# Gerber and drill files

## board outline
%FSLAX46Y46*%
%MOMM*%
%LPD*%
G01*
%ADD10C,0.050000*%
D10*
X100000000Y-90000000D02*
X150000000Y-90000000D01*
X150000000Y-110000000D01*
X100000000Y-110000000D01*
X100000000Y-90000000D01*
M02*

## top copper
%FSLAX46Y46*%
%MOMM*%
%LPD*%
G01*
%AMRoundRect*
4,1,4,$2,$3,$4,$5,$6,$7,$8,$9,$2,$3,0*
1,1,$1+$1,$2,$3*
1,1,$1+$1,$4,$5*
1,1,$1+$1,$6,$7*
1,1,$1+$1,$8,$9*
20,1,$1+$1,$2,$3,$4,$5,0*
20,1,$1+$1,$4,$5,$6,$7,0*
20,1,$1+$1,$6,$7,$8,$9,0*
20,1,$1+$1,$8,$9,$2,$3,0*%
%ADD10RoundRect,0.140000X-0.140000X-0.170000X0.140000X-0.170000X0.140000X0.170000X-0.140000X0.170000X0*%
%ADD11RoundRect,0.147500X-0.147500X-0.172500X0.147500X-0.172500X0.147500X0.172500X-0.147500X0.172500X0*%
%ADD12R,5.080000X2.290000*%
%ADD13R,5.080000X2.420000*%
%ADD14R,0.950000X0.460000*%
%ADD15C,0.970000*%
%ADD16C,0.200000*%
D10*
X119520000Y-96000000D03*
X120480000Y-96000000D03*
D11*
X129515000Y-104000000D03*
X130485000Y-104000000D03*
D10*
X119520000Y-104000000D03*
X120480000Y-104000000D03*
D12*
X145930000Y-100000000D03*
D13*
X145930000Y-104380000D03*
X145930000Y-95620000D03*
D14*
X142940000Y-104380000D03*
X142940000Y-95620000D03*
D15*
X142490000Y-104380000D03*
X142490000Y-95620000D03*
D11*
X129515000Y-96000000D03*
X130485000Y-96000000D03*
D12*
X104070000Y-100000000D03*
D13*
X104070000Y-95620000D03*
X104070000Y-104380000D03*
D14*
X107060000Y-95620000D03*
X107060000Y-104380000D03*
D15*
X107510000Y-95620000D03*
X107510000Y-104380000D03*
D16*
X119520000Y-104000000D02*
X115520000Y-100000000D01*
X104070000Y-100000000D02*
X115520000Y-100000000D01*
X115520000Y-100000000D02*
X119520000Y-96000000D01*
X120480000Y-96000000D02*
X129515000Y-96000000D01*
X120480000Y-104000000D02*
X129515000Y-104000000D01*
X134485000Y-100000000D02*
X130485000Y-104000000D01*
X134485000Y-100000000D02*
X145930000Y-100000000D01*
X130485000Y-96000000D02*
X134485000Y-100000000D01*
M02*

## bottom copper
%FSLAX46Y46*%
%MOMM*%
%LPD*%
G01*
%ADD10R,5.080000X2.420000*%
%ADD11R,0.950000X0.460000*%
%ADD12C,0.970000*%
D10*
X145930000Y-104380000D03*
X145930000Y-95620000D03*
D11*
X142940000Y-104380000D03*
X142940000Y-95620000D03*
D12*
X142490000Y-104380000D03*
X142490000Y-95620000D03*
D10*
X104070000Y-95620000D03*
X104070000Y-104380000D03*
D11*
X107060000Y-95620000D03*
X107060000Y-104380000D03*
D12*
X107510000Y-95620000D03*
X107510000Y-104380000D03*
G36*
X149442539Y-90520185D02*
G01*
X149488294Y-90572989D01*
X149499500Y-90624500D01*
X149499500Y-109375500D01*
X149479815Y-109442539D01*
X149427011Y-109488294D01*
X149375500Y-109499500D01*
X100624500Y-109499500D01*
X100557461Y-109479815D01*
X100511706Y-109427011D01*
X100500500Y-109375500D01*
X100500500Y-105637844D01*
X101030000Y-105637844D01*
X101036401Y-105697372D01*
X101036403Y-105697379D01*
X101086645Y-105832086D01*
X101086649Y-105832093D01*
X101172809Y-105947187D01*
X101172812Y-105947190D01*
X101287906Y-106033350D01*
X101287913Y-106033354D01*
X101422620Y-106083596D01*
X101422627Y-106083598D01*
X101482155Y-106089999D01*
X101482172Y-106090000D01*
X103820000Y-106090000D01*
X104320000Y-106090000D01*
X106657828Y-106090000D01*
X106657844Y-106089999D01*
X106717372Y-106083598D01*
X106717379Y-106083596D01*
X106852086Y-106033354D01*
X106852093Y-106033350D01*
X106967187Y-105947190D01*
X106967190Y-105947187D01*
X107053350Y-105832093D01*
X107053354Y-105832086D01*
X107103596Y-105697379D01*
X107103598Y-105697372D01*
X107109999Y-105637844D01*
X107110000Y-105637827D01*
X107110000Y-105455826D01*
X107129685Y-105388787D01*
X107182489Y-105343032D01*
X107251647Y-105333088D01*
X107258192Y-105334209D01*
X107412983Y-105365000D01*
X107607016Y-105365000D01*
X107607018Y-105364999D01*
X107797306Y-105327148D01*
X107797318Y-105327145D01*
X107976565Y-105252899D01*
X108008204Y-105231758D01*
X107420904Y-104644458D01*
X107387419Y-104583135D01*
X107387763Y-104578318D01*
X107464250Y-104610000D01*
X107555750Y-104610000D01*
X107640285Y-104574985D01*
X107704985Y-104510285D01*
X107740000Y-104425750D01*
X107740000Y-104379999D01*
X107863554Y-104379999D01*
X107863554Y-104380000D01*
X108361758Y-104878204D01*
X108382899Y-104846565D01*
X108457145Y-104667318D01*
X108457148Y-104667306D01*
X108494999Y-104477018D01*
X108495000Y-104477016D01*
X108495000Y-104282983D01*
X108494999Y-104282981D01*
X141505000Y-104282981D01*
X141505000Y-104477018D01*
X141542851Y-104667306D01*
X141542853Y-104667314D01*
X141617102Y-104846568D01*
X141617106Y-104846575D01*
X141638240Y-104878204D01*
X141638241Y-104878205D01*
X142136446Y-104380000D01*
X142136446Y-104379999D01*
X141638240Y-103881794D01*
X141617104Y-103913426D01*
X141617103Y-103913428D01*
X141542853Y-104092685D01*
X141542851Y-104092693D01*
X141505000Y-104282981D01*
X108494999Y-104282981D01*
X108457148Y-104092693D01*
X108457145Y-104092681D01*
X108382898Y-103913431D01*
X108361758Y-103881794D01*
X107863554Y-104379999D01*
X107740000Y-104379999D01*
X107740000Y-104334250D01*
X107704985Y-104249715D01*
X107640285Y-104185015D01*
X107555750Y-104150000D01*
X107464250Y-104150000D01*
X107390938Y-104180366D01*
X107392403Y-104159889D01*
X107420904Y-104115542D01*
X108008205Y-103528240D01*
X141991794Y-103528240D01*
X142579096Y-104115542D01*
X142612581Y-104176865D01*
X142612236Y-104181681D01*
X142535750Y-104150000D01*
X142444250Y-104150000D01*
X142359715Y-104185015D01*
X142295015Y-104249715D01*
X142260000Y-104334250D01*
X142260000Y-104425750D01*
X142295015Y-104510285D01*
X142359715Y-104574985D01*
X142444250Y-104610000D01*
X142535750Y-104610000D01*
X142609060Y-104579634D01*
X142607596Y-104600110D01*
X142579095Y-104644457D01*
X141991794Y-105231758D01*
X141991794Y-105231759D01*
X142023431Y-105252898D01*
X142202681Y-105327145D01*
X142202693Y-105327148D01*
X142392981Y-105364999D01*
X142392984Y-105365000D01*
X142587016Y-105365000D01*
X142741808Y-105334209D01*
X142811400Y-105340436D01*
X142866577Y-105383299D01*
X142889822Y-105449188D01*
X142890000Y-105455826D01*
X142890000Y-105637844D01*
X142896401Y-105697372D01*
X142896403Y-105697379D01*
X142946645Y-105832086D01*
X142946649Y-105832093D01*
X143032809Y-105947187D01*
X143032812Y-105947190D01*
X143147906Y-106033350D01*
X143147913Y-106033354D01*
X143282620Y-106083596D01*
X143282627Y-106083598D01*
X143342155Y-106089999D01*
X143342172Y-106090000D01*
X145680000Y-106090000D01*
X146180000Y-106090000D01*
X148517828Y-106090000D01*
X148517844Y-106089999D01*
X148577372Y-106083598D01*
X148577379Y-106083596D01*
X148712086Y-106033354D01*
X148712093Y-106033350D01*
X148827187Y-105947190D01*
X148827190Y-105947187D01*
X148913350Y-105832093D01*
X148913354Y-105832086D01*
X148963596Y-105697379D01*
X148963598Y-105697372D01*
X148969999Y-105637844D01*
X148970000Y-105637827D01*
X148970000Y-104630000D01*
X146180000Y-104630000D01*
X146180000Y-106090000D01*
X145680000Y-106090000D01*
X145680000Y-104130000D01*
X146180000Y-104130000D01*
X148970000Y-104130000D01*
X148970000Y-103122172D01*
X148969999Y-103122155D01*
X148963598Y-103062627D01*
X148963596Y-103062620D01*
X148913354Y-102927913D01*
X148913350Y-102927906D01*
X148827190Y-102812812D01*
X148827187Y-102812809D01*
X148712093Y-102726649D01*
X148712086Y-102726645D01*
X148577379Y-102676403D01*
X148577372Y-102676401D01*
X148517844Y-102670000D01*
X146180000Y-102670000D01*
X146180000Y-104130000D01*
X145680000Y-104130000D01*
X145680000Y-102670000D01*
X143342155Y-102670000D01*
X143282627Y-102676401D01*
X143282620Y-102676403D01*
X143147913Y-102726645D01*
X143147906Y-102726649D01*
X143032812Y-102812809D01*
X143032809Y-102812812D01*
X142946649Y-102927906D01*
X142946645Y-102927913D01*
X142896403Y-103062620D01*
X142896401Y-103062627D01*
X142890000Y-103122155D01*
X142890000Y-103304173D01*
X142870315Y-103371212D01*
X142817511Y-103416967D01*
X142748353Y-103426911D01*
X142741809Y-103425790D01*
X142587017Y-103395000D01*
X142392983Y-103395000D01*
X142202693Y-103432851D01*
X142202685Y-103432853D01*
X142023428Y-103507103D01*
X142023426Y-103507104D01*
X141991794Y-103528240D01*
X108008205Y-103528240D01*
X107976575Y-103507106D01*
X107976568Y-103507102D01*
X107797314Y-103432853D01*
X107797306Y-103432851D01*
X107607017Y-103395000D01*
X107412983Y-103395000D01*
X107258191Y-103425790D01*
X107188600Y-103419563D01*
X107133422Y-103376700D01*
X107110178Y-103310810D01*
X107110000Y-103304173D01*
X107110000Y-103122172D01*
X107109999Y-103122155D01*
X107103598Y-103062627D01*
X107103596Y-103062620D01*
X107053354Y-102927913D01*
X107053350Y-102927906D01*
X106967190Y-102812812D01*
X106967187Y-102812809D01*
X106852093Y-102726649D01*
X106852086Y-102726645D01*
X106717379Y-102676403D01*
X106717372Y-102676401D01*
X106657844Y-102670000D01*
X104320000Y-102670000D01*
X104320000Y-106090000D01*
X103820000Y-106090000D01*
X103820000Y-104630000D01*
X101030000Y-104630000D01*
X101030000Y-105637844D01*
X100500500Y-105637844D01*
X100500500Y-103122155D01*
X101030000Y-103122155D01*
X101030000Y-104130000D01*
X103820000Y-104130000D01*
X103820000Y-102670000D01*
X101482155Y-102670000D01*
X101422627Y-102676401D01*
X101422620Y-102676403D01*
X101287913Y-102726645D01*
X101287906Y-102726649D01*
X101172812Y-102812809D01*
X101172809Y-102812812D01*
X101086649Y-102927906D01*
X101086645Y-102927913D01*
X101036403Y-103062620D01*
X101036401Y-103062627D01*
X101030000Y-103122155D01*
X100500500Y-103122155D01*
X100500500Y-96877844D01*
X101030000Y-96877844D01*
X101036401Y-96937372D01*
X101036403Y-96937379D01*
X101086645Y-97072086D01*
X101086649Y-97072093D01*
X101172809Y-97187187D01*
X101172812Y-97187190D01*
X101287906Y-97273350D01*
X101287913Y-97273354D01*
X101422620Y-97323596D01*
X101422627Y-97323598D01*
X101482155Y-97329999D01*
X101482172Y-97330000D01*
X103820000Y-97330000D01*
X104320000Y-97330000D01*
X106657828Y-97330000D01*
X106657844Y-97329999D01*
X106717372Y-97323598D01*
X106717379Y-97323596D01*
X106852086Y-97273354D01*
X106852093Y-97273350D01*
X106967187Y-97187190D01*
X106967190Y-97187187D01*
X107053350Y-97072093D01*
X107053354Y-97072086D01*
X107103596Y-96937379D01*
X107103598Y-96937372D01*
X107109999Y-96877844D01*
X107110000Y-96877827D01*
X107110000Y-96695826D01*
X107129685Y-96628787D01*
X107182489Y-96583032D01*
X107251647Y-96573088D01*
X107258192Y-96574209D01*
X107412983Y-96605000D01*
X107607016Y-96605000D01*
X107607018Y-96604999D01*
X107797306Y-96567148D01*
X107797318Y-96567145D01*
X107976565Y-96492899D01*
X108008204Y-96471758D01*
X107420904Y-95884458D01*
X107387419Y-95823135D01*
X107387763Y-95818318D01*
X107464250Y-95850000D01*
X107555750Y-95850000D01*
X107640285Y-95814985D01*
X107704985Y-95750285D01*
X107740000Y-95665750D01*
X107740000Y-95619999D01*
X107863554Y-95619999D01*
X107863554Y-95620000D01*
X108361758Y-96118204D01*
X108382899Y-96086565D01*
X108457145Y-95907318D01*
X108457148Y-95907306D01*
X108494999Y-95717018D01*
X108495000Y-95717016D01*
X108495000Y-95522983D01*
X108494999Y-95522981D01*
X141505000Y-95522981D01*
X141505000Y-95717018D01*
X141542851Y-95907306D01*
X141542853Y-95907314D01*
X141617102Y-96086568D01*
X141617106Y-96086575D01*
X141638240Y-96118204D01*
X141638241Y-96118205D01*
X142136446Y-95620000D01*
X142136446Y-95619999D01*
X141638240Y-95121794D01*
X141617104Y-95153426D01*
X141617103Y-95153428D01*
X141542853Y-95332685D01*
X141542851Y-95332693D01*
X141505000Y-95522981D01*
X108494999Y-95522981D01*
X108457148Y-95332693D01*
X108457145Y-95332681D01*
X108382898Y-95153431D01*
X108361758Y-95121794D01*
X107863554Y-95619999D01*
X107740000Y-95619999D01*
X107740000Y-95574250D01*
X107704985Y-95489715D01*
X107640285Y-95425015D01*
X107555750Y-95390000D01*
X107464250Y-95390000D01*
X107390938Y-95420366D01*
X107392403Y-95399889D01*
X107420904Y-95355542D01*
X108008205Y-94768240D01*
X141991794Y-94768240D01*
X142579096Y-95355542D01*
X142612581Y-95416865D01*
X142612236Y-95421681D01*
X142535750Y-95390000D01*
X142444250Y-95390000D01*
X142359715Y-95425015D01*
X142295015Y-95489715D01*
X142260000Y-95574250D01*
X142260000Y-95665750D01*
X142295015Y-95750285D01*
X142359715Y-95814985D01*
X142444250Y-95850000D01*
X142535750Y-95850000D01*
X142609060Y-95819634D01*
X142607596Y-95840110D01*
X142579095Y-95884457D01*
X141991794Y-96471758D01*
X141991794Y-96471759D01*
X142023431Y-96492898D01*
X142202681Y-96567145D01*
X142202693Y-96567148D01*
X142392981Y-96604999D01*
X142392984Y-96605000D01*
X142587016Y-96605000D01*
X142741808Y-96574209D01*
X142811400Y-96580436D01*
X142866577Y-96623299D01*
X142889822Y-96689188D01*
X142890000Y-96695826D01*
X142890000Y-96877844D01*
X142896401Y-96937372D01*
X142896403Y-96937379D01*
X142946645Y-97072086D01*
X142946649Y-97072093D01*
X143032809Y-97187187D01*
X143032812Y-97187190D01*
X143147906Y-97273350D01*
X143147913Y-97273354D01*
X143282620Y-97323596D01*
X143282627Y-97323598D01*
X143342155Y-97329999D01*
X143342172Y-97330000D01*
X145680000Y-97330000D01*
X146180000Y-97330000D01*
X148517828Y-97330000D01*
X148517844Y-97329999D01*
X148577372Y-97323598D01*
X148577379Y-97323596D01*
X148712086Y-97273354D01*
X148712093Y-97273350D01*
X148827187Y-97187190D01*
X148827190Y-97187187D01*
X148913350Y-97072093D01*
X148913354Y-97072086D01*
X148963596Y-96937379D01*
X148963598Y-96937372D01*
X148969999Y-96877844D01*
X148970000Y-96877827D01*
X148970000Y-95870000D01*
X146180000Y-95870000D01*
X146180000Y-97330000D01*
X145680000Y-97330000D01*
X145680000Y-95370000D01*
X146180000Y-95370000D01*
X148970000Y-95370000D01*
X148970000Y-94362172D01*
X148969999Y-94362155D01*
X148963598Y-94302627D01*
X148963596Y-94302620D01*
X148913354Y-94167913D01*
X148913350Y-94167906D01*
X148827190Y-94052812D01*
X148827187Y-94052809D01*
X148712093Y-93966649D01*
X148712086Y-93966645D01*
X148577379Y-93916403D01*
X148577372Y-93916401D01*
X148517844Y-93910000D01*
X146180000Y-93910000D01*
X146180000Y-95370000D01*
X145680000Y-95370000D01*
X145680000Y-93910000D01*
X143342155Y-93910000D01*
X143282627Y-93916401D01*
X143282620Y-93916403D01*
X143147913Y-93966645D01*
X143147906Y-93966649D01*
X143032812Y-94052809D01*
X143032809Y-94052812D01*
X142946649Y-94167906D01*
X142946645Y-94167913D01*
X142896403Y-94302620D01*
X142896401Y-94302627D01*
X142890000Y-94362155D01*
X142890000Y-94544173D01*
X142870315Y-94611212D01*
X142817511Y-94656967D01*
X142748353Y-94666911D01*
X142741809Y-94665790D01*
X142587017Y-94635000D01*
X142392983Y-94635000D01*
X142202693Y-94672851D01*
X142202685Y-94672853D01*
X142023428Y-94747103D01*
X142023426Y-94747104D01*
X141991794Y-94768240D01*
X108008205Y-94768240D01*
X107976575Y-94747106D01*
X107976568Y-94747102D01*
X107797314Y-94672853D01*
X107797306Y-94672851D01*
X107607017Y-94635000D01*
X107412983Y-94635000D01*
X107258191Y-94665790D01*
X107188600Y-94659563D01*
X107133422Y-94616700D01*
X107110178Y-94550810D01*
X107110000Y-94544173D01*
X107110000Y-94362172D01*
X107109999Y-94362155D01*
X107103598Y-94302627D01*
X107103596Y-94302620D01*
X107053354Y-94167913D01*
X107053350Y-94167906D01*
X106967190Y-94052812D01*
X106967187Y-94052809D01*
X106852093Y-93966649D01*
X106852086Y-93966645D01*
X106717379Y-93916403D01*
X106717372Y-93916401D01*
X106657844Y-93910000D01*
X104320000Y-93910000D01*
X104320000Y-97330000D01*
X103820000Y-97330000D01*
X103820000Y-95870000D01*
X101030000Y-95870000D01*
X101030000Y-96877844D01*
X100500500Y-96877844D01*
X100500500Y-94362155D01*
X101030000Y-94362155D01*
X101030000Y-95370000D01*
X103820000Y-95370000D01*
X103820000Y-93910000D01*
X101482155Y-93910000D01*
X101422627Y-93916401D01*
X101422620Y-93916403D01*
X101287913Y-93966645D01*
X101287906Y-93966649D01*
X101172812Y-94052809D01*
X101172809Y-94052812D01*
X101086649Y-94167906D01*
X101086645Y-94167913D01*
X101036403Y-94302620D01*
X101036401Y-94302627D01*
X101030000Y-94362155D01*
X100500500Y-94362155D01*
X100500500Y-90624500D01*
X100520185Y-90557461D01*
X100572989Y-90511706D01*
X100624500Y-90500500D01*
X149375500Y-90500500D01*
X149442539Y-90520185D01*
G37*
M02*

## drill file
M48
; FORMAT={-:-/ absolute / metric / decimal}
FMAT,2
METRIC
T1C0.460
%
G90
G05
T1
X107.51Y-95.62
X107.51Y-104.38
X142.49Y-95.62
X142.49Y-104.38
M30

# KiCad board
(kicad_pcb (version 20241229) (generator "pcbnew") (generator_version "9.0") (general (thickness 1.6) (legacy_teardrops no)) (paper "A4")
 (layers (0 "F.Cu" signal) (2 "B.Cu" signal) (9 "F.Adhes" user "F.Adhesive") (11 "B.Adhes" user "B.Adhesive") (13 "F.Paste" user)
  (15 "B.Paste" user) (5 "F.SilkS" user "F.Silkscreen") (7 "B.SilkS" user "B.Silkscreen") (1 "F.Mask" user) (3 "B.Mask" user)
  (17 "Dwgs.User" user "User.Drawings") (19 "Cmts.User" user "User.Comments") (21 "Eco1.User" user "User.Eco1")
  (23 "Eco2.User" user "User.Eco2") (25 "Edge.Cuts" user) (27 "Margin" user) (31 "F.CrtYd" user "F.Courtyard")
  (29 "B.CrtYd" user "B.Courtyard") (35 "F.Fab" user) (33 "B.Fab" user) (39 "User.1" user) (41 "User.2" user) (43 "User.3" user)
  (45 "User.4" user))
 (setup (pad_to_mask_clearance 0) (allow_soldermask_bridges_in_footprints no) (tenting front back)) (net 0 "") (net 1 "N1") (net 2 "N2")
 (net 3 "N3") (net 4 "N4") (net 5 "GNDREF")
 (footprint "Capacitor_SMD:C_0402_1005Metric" (layer "F.Cu") (at 120 96)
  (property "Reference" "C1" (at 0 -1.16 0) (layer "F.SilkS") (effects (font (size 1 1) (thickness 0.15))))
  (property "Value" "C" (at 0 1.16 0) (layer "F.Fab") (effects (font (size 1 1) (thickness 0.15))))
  (pad "1" smd roundrect (at -0.48 0) (size 0.56 0.62) (layers "F.Cu" "F.Mask" "F.Paste") (roundrect_rratio 0.25) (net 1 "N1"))
  (pad "2" smd roundrect (at 0.48 0) (size 0.56 0.62) (layers "F.Cu" "F.Mask" "F.Paste") (roundrect_rratio 0.25) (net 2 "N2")))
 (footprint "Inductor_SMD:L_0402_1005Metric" (layer "F.Cu") (at 130 104)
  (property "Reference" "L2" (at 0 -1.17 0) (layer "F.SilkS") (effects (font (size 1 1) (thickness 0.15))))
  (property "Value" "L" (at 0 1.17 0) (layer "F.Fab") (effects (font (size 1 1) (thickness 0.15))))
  (pad "1" smd roundrect (at -0.485 0) (size 0.59 0.64) (layers "F.Cu" "F.Mask" "F.Paste") (roundrect_rratio 0.25) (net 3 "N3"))
  (pad "2" smd roundrect (at 0.485 0) (size 0.59 0.64) (layers "F.Cu" "F.Mask" "F.Paste") (roundrect_rratio 0.25) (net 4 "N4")))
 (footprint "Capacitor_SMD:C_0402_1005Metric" (layer "F.Cu") (at 120 104)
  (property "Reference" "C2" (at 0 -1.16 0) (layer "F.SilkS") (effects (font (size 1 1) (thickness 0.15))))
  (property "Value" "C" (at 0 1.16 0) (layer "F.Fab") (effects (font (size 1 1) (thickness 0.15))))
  (pad "1" smd roundrect (at -0.48 0) (size 0.56 0.62) (layers "F.Cu" "F.Mask" "F.Paste") (roundrect_rratio 0.25) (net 1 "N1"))
  (pad "2" smd roundrect (at 0.48 0) (size 0.56 0.62) (layers "F.Cu" "F.Mask" "F.Paste") (roundrect_rratio 0.25) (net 3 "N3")))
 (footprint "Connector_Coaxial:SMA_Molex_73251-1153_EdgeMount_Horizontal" (layer "F.Cu") (at 144.21 100 180)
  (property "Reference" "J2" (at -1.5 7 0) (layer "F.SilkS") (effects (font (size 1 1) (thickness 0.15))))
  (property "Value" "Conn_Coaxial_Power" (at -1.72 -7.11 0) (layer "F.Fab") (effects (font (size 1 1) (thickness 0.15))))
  (pad "1" smd rect (at -1.72 0 180) (size 5.08 2.29) (layers "F.Cu" "F.Mask" "F.Paste") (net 4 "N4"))
  (pad "2" smd rect (at -1.72 -4.38 180) (size 5.08 2.42) (layers "F.Cu" "F.Mask" "F.Paste") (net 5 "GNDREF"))
  (pad "2" smd rect (at -1.72 -4.38 180) (size 5.08 2.42) (layers "B.Cu" "B.Mask" "B.Paste") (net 5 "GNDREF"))
  (pad "2" smd rect (at -1.72 4.38 180) (size 5.08 2.42) (layers "F.Cu" "F.Mask" "F.Paste") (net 5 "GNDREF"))
  (pad "2" smd rect (at -1.72 4.38 180) (size 5.08 2.42) (layers "B.Cu" "B.Mask" "B.Paste") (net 5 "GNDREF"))
  (pad "2" smd rect (at 1.27 -4.38 180) (size 0.95 0.46) (layers "F.Cu") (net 5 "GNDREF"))
  (pad "2" smd rect (at 1.27 -4.38 180) (size 0.95 0.46) (layers "B.Cu") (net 5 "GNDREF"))
  (pad "2" smd rect (at 1.27 4.38 180) (size 0.95 0.46) (layers "F.Cu") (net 5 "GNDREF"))
  (pad "2" smd rect (at 1.27 4.38 180) (size 0.95 0.46) (layers "B.Cu") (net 5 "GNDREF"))
  (pad "2" thru_hole circle (at 1.72 -4.38 180) (size 0.97 0.97) (drill 0.46) (layers "*.Cu") (remove_unused_layers no) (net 5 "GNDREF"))
  (pad "2" thru_hole circle (at 1.72 4.38 180) (size 0.97 0.97) (drill 0.46) (layers "*.Cu") (remove_unused_layers no) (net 5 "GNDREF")))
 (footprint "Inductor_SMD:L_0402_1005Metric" (layer "F.Cu") (at 130 96)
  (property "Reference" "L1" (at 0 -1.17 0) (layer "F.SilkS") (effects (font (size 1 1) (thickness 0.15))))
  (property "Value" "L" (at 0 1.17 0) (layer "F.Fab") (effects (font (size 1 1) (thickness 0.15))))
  (pad "1" smd roundrect (at -0.485 0) (size 0.59 0.64) (layers "F.Cu" "F.Mask" "F.Paste") (roundrect_rratio 0.25) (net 2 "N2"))
  (pad "2" smd roundrect (at 0.485 0) (size 0.59 0.64) (layers "F.Cu" "F.Mask" "F.Paste") (roundrect_rratio 0.25) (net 4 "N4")))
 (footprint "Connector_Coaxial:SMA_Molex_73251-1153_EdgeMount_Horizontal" (layer "F.Cu") (at 105.79 100)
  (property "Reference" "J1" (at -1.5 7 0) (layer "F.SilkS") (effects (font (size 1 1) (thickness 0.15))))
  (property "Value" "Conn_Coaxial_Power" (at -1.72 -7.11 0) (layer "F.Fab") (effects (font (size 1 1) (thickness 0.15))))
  (pad "1" smd rect (at -1.72 0) (size 5.08 2.29) (layers "F.Cu" "F.Mask" "F.Paste") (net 1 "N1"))
  (pad "2" smd rect (at -1.72 -4.38) (size 5.08 2.42) (layers "F.Cu" "F.Mask" "F.Paste") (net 5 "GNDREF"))
  (pad "2" smd rect (at -1.72 -4.38) (size 5.08 2.42) (layers "B.Cu" "B.Mask" "B.Paste") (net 5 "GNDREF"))
  (pad "2" smd rect (at -1.72 4.38) (size 5.08 2.42) (layers "F.Cu" "F.Mask" "F.Paste") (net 5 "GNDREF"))
  (pad "2" smd rect (at -1.72 4.38) (size 5.08 2.42) (layers "B.Cu" "B.Mask" "B.Paste") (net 5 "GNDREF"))
  (pad "2" smd rect (at 1.27 -4.38) (size 0.95 0.46) (layers "F.Cu") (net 5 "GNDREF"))
  (pad "2" smd rect (at 1.27 -4.38) (size 0.95 0.46) (layers "B.Cu") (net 5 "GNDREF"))
  (pad "2" smd rect (at 1.27 4.38) (size 0.95 0.46) (layers "F.Cu") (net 5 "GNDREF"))
  (pad "2" smd rect (at 1.27 4.38) (size 0.95 0.46) (layers "B.Cu") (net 5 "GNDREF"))
  (pad "2" thru_hole circle (at 1.72 -4.38) (size 0.97 0.97) (drill 0.46) (layers "*.Cu") (remove_unused_layers no) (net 5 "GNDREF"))
  (pad "2" thru_hole circle (at 1.72 4.38) (size 0.97 0.97) (drill 0.46) (layers "*.Cu") (remove_unused_layers no) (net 5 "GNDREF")))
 (gr_rect (start 100 90) (end 150 110) (stroke (width 0.05) (type default)) (fill no) (layer "Edge.Cuts"))
 (segment (start 119.52 104) (end 115.52 100) (width 0.2) (layer "F.Cu") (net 1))
 (segment (start 104.07 100) (end 115.52 100) (width 0.2) (layer "F.Cu") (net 1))
 (segment (start 115.52 100) (end 119.52 96) (width 0.2) (layer "F.Cu") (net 1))
 (segment (start 120.48 96) (end 129.515 96) (width 0.2) (layer "F.Cu") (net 2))
 (segment (start 120.48 104) (end 129.515 104) (width 0.2) (layer "F.Cu") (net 3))
 (segment (start 134.485 100) (end 130.485 104) (width 0.2) (layer "F.Cu") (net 4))
 (segment (start 134.485 100) (end 145.93 100) (width 0.2) (layer "F.Cu") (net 4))
 (segment (start 130.485 96) (end 134.485 100) (width 0.2) (layer "F.Cu") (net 4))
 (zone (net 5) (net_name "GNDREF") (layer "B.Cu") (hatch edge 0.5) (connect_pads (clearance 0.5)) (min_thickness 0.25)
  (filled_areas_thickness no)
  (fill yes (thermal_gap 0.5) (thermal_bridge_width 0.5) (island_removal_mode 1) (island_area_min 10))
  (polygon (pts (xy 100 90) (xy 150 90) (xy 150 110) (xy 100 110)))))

